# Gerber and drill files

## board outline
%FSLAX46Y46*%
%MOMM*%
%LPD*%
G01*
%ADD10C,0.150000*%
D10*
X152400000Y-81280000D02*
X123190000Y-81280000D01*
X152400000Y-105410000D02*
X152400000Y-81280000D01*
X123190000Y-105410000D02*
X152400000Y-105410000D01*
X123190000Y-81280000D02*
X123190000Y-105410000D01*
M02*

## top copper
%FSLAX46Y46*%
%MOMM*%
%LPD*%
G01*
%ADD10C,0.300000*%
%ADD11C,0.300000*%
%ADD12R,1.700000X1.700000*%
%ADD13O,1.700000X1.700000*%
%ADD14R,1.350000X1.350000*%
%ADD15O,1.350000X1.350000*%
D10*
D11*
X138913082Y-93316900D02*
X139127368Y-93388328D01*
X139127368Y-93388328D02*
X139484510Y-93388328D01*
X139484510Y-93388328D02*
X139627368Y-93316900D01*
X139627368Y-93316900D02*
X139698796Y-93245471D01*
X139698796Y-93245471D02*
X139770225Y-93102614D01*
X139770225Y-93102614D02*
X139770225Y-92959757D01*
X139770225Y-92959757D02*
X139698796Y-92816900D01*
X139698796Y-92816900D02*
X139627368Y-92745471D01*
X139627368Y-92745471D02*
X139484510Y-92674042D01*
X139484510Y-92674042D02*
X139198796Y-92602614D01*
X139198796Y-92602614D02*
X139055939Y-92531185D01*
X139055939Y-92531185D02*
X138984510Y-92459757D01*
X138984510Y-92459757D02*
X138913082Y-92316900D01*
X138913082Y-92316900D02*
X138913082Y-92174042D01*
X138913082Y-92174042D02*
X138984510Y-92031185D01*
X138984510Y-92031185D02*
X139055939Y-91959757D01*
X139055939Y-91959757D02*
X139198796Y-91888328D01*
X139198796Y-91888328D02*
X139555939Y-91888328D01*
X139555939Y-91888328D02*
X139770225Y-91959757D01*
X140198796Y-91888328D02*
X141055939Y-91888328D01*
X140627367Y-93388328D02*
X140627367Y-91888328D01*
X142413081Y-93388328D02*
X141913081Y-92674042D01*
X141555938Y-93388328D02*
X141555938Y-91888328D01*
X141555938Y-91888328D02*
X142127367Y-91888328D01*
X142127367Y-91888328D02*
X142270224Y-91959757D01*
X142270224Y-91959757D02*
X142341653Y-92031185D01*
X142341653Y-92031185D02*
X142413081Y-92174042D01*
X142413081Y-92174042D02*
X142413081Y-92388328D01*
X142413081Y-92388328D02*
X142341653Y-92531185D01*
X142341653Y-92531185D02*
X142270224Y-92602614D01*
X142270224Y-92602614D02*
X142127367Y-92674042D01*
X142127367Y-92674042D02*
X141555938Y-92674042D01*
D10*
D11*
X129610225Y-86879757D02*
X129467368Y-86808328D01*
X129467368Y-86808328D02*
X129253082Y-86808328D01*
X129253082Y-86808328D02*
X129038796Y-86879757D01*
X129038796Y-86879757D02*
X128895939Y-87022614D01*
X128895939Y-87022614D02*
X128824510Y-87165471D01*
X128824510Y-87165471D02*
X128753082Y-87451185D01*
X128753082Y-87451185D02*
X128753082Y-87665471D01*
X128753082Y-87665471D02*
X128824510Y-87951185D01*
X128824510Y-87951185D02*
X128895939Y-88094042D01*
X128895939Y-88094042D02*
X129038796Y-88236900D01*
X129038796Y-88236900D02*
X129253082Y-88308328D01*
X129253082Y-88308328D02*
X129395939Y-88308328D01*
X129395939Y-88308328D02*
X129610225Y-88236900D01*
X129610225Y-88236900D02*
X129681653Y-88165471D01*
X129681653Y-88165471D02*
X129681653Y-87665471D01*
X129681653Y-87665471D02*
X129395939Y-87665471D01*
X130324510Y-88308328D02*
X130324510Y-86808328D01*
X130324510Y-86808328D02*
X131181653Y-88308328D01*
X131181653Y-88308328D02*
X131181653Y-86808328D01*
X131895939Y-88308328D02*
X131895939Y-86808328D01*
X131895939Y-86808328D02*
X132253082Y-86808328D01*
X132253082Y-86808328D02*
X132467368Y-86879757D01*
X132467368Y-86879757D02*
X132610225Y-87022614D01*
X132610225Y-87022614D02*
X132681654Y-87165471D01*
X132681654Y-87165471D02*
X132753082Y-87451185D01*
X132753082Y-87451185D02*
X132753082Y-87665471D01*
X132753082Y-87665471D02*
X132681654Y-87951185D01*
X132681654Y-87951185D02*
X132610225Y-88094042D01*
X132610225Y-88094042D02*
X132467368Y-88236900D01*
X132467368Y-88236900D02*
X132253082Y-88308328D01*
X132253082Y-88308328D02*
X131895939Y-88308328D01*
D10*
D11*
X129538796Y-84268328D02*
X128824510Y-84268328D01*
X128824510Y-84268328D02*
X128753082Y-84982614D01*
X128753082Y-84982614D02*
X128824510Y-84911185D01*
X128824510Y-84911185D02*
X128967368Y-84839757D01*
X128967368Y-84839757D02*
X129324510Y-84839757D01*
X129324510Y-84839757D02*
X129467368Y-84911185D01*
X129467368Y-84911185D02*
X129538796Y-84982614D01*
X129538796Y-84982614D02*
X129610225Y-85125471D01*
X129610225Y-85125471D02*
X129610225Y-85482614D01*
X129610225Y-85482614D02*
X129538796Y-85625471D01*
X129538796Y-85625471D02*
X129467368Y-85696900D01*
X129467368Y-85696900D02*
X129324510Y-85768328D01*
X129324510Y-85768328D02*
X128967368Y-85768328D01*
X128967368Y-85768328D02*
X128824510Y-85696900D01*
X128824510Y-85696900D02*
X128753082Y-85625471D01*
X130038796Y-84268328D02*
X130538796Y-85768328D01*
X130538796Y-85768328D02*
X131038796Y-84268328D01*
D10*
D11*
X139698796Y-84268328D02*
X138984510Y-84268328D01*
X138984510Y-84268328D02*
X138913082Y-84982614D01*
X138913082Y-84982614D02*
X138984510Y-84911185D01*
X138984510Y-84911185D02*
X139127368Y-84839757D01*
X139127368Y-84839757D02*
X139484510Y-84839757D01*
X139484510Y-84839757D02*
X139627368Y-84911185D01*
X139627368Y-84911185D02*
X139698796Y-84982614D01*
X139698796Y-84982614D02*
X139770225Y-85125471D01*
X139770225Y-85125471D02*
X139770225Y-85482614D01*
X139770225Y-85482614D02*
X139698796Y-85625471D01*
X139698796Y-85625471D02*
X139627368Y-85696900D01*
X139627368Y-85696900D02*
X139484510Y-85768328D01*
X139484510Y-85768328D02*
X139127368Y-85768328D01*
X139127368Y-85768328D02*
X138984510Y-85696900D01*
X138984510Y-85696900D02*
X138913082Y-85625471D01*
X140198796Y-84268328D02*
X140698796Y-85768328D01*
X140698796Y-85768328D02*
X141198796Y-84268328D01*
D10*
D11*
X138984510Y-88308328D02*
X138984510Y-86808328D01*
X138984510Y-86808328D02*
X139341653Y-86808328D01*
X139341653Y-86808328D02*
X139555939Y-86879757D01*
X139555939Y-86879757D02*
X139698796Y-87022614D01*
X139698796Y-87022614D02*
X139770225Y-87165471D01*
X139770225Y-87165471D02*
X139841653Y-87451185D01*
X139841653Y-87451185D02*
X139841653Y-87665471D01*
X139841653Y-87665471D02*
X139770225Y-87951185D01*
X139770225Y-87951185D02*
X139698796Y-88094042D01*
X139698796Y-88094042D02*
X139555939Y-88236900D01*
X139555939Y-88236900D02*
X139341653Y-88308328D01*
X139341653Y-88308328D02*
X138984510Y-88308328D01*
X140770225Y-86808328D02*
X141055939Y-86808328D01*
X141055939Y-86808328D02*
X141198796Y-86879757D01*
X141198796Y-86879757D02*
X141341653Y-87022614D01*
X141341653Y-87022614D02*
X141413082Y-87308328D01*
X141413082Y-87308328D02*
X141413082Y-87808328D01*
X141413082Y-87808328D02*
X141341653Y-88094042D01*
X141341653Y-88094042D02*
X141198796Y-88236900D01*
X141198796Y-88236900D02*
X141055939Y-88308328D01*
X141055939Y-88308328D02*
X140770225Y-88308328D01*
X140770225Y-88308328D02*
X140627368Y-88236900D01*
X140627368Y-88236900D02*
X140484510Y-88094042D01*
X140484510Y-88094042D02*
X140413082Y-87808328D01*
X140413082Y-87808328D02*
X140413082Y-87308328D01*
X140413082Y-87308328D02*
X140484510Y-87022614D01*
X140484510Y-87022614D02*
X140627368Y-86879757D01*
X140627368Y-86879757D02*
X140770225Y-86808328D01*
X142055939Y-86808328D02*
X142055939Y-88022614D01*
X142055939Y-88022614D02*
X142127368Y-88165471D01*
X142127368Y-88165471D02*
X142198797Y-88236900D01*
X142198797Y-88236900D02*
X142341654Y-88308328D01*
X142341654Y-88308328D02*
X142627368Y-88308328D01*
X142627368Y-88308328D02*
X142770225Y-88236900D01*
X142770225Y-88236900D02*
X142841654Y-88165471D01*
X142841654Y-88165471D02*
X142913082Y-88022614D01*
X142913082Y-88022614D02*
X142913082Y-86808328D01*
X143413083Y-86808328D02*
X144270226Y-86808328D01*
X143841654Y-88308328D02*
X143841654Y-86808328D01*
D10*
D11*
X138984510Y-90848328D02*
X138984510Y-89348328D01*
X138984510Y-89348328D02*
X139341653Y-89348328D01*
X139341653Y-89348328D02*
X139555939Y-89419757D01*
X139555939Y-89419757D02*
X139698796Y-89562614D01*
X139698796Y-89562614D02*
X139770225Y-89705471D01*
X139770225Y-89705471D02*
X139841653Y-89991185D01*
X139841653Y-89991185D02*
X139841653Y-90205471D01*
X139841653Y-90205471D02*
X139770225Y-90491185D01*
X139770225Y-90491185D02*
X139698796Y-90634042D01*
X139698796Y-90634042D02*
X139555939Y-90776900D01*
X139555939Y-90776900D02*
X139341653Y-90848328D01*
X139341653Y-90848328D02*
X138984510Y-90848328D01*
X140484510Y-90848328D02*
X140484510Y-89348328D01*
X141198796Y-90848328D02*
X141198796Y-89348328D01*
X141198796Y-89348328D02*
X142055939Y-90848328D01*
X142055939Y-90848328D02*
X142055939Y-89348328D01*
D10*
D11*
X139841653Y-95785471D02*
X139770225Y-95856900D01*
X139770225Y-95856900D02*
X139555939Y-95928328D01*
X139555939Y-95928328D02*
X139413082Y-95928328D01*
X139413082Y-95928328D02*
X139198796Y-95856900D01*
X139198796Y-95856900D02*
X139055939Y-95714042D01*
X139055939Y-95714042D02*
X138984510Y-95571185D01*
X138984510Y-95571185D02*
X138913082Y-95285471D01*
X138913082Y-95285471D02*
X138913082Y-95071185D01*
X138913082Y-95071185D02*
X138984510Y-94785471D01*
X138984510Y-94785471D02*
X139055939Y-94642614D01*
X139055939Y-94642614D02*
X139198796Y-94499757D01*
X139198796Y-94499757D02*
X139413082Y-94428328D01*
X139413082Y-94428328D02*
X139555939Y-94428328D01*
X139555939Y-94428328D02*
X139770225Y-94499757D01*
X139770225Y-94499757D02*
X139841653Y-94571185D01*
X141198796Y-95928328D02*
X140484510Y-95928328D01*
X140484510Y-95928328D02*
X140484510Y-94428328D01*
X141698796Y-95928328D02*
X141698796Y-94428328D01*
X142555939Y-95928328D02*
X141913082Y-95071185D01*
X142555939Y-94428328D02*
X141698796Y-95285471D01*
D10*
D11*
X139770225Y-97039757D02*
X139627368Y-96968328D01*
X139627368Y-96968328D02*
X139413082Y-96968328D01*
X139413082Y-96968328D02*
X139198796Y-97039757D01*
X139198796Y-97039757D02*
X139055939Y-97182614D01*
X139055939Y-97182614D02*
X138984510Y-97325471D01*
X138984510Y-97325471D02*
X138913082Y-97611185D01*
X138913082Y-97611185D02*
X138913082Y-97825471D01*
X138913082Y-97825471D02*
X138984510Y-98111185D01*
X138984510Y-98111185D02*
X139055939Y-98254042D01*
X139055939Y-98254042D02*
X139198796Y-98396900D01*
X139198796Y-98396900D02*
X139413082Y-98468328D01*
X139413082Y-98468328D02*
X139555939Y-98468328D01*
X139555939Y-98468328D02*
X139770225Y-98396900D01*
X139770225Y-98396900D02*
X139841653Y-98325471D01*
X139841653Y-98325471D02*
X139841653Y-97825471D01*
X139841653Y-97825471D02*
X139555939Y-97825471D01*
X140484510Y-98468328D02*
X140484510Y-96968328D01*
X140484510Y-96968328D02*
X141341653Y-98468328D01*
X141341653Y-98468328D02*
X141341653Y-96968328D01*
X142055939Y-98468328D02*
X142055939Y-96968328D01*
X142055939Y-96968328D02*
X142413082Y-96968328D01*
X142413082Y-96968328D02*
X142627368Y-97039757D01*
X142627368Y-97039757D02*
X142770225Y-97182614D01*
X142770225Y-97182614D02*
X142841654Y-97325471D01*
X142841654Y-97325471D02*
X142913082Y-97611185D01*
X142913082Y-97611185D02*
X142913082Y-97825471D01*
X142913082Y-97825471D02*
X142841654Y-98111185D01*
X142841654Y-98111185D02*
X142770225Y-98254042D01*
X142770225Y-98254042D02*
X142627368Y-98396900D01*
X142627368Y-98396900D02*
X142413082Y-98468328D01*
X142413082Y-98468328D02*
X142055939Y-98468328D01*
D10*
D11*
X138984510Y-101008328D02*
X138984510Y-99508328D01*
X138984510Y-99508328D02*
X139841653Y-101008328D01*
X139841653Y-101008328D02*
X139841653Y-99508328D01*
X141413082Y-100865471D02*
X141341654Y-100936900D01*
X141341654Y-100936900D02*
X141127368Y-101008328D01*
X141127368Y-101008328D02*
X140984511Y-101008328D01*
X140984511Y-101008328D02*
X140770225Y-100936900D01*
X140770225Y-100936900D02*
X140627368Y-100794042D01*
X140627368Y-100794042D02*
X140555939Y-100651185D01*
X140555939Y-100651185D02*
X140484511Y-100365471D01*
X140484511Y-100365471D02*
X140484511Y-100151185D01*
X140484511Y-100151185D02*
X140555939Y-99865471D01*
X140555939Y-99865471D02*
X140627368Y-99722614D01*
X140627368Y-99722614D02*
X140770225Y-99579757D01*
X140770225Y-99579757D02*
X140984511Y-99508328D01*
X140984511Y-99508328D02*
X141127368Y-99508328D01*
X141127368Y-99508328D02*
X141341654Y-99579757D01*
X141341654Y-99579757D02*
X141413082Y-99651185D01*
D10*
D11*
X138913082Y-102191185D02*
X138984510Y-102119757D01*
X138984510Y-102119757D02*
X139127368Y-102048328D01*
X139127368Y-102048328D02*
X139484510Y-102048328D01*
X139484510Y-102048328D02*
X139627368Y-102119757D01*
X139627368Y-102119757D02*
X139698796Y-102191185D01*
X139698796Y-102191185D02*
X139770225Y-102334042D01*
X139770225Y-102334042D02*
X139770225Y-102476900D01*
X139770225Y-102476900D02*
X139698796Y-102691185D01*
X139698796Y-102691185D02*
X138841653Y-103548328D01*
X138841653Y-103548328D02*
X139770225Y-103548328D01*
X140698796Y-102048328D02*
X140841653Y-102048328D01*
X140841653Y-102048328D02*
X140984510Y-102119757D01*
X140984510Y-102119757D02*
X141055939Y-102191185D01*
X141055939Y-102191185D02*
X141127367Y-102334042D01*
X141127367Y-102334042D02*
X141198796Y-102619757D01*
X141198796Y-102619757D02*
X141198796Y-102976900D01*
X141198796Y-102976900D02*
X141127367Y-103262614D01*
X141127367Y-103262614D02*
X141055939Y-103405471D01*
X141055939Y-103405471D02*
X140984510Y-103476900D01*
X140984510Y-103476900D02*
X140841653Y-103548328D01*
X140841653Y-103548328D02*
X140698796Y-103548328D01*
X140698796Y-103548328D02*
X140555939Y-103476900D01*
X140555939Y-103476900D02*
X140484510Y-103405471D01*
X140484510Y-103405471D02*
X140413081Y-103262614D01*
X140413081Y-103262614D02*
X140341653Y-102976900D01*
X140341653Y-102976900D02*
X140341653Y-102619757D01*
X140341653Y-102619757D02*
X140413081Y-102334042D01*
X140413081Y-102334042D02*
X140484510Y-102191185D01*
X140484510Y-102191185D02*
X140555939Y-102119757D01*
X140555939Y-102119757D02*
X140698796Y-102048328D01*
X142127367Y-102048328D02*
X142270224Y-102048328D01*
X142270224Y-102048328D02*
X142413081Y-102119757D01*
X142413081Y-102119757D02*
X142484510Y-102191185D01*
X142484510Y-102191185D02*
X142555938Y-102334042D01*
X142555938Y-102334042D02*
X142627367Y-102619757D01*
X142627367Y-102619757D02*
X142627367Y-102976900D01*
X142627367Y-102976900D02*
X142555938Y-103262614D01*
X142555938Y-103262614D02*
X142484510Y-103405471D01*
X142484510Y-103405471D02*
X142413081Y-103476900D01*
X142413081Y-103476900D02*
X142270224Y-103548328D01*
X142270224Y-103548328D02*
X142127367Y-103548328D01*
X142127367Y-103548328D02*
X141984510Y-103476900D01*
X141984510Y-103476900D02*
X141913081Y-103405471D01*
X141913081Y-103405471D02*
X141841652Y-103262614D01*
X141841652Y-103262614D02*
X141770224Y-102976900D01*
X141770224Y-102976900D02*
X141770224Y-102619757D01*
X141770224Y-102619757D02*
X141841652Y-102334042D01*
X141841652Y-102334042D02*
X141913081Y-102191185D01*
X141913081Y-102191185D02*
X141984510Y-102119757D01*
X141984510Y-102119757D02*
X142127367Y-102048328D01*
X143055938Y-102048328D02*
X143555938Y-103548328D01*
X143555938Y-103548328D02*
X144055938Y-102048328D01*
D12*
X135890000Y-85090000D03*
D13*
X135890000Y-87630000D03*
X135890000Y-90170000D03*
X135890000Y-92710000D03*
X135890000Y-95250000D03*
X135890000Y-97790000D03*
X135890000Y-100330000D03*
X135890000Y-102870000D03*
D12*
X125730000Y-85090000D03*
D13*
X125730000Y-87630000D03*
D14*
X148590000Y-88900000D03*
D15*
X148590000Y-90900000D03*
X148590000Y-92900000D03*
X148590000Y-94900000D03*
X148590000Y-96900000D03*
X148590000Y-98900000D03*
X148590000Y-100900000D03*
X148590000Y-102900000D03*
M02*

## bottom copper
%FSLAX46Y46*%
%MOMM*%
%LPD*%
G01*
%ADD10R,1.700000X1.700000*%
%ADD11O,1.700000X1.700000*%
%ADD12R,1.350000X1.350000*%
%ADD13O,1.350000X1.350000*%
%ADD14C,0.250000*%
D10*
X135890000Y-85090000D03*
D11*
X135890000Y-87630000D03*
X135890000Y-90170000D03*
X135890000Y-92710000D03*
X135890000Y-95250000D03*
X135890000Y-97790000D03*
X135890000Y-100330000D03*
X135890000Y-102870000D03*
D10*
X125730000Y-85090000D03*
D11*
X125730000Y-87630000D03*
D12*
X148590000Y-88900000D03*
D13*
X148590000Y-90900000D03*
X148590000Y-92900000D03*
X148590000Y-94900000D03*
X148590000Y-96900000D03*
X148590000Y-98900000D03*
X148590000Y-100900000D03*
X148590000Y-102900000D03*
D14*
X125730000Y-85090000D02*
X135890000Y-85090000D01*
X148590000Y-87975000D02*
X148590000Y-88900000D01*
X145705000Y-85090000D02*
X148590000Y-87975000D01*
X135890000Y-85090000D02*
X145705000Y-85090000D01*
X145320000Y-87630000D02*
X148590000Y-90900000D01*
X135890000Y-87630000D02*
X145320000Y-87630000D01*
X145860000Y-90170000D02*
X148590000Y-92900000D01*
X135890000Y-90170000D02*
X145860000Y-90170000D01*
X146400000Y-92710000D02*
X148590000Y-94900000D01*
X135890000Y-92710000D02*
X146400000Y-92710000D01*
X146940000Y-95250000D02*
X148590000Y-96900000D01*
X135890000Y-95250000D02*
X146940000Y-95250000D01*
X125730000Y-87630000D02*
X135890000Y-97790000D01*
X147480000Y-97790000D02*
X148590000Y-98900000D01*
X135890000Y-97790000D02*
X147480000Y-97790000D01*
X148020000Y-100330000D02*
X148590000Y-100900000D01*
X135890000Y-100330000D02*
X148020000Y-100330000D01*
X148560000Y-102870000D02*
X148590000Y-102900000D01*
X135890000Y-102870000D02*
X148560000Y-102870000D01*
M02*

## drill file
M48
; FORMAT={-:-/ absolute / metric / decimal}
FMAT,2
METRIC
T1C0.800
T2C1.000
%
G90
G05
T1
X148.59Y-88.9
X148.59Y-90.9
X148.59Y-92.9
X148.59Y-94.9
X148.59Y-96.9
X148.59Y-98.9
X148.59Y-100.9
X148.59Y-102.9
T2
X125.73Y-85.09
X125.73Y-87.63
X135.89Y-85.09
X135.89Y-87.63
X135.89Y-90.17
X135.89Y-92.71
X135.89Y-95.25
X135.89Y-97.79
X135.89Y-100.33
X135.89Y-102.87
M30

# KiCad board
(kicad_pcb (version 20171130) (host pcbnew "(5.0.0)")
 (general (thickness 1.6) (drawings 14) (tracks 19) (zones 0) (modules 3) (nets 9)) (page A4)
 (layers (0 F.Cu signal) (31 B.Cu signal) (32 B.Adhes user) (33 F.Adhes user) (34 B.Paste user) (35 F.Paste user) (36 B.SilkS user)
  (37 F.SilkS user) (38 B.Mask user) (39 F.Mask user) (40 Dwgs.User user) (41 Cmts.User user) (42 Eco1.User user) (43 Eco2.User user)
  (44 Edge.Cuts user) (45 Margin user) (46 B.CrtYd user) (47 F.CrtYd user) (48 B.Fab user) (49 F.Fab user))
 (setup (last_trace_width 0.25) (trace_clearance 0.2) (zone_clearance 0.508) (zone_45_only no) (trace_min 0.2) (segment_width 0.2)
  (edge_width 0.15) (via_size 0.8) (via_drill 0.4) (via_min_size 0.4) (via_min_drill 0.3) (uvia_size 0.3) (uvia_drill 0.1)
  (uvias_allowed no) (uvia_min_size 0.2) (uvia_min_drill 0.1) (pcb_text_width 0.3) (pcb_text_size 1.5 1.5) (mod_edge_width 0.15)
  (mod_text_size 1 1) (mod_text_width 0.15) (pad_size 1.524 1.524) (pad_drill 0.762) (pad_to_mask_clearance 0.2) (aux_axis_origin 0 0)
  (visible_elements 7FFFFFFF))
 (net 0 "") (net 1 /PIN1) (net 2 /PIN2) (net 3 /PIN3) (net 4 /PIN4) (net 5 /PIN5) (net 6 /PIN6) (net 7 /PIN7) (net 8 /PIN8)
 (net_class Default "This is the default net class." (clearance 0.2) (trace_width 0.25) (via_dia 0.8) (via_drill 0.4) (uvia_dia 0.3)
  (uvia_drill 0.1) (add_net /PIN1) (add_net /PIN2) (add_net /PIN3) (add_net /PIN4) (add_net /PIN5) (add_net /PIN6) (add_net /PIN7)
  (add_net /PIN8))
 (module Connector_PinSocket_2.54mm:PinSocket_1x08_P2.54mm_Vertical (layer F.Cu) (at 135.89 85.09)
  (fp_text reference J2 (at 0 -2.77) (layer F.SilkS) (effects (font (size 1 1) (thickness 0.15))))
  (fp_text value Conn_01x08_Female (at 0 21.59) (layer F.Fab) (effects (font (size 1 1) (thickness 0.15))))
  (pad 1 thru_hole rect (at 0 0) (size 1.7 1.7) (drill 1) (layers *.Cu *.Mask) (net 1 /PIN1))
  (pad 2 thru_hole oval (at 0 2.54) (size 1.7 1.7) (drill 1) (layers *.Cu *.Mask) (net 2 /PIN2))
  (pad 3 thru_hole oval (at 0 5.08) (size 1.7 1.7) (drill 1) (layers *.Cu *.Mask) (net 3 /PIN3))
  (pad 4 thru_hole oval (at 0 7.62) (size 1.7 1.7) (drill 1) (layers *.Cu *.Mask) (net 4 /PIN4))
  (pad 5 thru_hole oval (at 0 10.16) (size 1.7 1.7) (drill 1) (layers *.Cu *.Mask) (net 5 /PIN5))
  (pad 6 thru_hole oval (at 0 12.7) (size 1.7 1.7) (drill 1) (layers *.Cu *.Mask) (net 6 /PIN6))
  (pad 7 thru_hole oval (at 0 15.24) (size 1.7 1.7) (drill 1) (layers *.Cu *.Mask) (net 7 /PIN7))
  (pad 8 thru_hole oval (at 0 17.78) (size 1.7 1.7) (drill 1) (layers *.Cu *.Mask) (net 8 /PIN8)))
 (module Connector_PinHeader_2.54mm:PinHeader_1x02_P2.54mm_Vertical (layer F.Cu) (at 125.73 85.09)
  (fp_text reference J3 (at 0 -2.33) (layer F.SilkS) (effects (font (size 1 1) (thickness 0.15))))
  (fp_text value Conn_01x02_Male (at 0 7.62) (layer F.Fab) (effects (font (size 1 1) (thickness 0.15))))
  (pad 1 thru_hole rect (at 0 0) (size 1.7 1.7) (drill 1) (layers *.Cu *.Mask) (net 1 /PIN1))
  (pad 2 thru_hole oval (at 0 2.54) (size 1.7 1.7) (drill 1) (layers *.Cu *.Mask) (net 6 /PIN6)))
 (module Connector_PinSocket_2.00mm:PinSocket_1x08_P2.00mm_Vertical (layer F.Cu) (at 148.59 88.9)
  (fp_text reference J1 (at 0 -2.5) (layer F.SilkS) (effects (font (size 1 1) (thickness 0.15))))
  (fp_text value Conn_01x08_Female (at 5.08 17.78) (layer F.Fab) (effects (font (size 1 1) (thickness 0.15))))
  (pad 1 thru_hole rect (at 0 0) (size 1.35 1.35) (drill 0.8) (layers *.Cu *.Mask) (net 1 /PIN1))
  (pad 2 thru_hole oval (at 0 2) (size 1.35 1.35) (drill 0.8) (layers *.Cu *.Mask) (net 2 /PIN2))
  (pad 3 thru_hole oval (at 0 4) (size 1.35 1.35) (drill 0.8) (layers *.Cu *.Mask) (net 3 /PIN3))
  (pad 4 thru_hole oval (at 0 6) (size 1.35 1.35) (drill 0.8) (layers *.Cu *.Mask) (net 4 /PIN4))
  (pad 5 thru_hole oval (at 0 8) (size 1.35 1.35) (drill 0.8) (layers *.Cu *.Mask) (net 5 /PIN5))
  (pad 6 thru_hole oval (at 0 10) (size 1.35 1.35) (drill 0.8) (layers *.Cu *.Mask) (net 6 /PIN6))
  (pad 7 thru_hole oval (at 0 12) (size 1.35 1.35) (drill 0.8) (layers *.Cu *.Mask) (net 7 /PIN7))
  (pad 8 thru_hole oval (at 0 14) (size 1.35 1.35) (drill 0.8) (layers *.Cu *.Mask) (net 8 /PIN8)))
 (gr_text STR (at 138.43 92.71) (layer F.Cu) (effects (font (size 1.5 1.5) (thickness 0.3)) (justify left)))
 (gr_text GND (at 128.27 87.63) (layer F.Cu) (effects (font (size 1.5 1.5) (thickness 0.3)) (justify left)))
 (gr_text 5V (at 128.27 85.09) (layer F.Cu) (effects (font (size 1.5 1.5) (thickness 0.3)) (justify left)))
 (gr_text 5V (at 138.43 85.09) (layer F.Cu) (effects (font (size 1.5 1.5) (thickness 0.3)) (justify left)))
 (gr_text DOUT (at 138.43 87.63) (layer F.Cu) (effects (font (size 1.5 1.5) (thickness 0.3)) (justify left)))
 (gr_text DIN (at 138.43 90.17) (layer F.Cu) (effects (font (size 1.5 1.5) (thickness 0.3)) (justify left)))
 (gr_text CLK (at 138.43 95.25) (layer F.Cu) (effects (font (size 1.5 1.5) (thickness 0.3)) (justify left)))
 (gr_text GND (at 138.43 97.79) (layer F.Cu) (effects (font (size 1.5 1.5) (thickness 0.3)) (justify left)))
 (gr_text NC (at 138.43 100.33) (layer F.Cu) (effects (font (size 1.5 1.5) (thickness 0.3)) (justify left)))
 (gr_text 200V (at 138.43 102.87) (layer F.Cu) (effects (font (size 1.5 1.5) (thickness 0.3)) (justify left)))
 (gr_line (start 152.4 81.28) (end 123.19 81.28) (layer Edge.Cuts) (width 0.15))
 (gr_line (start 152.4 105.41) (end 152.4 81.28) (layer Edge.Cuts) (width 0.15))
 (gr_line (start 123.19 105.41) (end 152.4 105.41) (layer Edge.Cuts) (width 0.15))
 (gr_line (start 123.19 81.28) (end 123.19 105.41) (layer Edge.Cuts) (width 0.15))
 (segment (start 125.73 85.09) (end 135.89 85.09) (width 0.25) (layer B.Cu) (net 1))
 (segment (start 148.59 87.975) (end 148.59 88.9) (width 0.25) (layer B.Cu) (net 1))
 (segment (start 145.705 85.09) (end 148.59 87.975) (width 0.25) (layer B.Cu) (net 1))
 (segment (start 135.89 85.09) (end 145.705 85.09) (width 0.25) (layer B.Cu) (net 1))
 (segment (start 145.32 87.63) (end 148.59 90.9) (width 0.25) (layer B.Cu) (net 2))
 (segment (start 135.89 87.63) (end 145.32 87.63) (width 0.25) (layer B.Cu) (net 2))
 (segment (start 145.86 90.17) (end 148.59 92.9) (width 0.25) (layer B.Cu) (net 3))
 (segment (start 135.89 90.17) (end 145.86 90.17) (width 0.25) (layer B.Cu) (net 3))
 (segment (start 146.4 92.71) (end 148.59 94.9) (width 0.25) (layer B.Cu) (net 4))
 (segment (start 135.89 92.71) (end 146.4 92.71) (width 0.25) (layer B.Cu) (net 4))
 (segment (start 146.94 95.25) (end 148.59 96.9) (width 0.25) (layer B.Cu) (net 5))
 (segment (start 135.89 95.25) (end 146.94 95.25) (width 0.25) (layer B.Cu) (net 5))
 (segment (start 125.73 87.63) (end 135.89 97.79) (width 0.25) (layer B.Cu) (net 6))
 (segment (start 147.48 97.79) (end 148.59 98.9) (width 0.25) (layer B.Cu) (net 6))
 (segment (start 135.89 97.79) (end 147.48 97.79) (width 0.25) (layer B.Cu) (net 6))
 (segment (start 148.02 100.33) (end 148.59 100.9) (width 0.25) (layer B.Cu) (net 7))
 (segment (start 135.89 100.33) (end 148.02 100.33) (width 0.25) (layer B.Cu) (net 7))
 (segment (start 148.56 102.87) (end 148.59 102.9) (width 0.25) (layer B.Cu) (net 8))
 (segment (start 135.89 102.87) (end 148.56 102.87) (width 0.25) (layer B.Cu) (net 8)))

